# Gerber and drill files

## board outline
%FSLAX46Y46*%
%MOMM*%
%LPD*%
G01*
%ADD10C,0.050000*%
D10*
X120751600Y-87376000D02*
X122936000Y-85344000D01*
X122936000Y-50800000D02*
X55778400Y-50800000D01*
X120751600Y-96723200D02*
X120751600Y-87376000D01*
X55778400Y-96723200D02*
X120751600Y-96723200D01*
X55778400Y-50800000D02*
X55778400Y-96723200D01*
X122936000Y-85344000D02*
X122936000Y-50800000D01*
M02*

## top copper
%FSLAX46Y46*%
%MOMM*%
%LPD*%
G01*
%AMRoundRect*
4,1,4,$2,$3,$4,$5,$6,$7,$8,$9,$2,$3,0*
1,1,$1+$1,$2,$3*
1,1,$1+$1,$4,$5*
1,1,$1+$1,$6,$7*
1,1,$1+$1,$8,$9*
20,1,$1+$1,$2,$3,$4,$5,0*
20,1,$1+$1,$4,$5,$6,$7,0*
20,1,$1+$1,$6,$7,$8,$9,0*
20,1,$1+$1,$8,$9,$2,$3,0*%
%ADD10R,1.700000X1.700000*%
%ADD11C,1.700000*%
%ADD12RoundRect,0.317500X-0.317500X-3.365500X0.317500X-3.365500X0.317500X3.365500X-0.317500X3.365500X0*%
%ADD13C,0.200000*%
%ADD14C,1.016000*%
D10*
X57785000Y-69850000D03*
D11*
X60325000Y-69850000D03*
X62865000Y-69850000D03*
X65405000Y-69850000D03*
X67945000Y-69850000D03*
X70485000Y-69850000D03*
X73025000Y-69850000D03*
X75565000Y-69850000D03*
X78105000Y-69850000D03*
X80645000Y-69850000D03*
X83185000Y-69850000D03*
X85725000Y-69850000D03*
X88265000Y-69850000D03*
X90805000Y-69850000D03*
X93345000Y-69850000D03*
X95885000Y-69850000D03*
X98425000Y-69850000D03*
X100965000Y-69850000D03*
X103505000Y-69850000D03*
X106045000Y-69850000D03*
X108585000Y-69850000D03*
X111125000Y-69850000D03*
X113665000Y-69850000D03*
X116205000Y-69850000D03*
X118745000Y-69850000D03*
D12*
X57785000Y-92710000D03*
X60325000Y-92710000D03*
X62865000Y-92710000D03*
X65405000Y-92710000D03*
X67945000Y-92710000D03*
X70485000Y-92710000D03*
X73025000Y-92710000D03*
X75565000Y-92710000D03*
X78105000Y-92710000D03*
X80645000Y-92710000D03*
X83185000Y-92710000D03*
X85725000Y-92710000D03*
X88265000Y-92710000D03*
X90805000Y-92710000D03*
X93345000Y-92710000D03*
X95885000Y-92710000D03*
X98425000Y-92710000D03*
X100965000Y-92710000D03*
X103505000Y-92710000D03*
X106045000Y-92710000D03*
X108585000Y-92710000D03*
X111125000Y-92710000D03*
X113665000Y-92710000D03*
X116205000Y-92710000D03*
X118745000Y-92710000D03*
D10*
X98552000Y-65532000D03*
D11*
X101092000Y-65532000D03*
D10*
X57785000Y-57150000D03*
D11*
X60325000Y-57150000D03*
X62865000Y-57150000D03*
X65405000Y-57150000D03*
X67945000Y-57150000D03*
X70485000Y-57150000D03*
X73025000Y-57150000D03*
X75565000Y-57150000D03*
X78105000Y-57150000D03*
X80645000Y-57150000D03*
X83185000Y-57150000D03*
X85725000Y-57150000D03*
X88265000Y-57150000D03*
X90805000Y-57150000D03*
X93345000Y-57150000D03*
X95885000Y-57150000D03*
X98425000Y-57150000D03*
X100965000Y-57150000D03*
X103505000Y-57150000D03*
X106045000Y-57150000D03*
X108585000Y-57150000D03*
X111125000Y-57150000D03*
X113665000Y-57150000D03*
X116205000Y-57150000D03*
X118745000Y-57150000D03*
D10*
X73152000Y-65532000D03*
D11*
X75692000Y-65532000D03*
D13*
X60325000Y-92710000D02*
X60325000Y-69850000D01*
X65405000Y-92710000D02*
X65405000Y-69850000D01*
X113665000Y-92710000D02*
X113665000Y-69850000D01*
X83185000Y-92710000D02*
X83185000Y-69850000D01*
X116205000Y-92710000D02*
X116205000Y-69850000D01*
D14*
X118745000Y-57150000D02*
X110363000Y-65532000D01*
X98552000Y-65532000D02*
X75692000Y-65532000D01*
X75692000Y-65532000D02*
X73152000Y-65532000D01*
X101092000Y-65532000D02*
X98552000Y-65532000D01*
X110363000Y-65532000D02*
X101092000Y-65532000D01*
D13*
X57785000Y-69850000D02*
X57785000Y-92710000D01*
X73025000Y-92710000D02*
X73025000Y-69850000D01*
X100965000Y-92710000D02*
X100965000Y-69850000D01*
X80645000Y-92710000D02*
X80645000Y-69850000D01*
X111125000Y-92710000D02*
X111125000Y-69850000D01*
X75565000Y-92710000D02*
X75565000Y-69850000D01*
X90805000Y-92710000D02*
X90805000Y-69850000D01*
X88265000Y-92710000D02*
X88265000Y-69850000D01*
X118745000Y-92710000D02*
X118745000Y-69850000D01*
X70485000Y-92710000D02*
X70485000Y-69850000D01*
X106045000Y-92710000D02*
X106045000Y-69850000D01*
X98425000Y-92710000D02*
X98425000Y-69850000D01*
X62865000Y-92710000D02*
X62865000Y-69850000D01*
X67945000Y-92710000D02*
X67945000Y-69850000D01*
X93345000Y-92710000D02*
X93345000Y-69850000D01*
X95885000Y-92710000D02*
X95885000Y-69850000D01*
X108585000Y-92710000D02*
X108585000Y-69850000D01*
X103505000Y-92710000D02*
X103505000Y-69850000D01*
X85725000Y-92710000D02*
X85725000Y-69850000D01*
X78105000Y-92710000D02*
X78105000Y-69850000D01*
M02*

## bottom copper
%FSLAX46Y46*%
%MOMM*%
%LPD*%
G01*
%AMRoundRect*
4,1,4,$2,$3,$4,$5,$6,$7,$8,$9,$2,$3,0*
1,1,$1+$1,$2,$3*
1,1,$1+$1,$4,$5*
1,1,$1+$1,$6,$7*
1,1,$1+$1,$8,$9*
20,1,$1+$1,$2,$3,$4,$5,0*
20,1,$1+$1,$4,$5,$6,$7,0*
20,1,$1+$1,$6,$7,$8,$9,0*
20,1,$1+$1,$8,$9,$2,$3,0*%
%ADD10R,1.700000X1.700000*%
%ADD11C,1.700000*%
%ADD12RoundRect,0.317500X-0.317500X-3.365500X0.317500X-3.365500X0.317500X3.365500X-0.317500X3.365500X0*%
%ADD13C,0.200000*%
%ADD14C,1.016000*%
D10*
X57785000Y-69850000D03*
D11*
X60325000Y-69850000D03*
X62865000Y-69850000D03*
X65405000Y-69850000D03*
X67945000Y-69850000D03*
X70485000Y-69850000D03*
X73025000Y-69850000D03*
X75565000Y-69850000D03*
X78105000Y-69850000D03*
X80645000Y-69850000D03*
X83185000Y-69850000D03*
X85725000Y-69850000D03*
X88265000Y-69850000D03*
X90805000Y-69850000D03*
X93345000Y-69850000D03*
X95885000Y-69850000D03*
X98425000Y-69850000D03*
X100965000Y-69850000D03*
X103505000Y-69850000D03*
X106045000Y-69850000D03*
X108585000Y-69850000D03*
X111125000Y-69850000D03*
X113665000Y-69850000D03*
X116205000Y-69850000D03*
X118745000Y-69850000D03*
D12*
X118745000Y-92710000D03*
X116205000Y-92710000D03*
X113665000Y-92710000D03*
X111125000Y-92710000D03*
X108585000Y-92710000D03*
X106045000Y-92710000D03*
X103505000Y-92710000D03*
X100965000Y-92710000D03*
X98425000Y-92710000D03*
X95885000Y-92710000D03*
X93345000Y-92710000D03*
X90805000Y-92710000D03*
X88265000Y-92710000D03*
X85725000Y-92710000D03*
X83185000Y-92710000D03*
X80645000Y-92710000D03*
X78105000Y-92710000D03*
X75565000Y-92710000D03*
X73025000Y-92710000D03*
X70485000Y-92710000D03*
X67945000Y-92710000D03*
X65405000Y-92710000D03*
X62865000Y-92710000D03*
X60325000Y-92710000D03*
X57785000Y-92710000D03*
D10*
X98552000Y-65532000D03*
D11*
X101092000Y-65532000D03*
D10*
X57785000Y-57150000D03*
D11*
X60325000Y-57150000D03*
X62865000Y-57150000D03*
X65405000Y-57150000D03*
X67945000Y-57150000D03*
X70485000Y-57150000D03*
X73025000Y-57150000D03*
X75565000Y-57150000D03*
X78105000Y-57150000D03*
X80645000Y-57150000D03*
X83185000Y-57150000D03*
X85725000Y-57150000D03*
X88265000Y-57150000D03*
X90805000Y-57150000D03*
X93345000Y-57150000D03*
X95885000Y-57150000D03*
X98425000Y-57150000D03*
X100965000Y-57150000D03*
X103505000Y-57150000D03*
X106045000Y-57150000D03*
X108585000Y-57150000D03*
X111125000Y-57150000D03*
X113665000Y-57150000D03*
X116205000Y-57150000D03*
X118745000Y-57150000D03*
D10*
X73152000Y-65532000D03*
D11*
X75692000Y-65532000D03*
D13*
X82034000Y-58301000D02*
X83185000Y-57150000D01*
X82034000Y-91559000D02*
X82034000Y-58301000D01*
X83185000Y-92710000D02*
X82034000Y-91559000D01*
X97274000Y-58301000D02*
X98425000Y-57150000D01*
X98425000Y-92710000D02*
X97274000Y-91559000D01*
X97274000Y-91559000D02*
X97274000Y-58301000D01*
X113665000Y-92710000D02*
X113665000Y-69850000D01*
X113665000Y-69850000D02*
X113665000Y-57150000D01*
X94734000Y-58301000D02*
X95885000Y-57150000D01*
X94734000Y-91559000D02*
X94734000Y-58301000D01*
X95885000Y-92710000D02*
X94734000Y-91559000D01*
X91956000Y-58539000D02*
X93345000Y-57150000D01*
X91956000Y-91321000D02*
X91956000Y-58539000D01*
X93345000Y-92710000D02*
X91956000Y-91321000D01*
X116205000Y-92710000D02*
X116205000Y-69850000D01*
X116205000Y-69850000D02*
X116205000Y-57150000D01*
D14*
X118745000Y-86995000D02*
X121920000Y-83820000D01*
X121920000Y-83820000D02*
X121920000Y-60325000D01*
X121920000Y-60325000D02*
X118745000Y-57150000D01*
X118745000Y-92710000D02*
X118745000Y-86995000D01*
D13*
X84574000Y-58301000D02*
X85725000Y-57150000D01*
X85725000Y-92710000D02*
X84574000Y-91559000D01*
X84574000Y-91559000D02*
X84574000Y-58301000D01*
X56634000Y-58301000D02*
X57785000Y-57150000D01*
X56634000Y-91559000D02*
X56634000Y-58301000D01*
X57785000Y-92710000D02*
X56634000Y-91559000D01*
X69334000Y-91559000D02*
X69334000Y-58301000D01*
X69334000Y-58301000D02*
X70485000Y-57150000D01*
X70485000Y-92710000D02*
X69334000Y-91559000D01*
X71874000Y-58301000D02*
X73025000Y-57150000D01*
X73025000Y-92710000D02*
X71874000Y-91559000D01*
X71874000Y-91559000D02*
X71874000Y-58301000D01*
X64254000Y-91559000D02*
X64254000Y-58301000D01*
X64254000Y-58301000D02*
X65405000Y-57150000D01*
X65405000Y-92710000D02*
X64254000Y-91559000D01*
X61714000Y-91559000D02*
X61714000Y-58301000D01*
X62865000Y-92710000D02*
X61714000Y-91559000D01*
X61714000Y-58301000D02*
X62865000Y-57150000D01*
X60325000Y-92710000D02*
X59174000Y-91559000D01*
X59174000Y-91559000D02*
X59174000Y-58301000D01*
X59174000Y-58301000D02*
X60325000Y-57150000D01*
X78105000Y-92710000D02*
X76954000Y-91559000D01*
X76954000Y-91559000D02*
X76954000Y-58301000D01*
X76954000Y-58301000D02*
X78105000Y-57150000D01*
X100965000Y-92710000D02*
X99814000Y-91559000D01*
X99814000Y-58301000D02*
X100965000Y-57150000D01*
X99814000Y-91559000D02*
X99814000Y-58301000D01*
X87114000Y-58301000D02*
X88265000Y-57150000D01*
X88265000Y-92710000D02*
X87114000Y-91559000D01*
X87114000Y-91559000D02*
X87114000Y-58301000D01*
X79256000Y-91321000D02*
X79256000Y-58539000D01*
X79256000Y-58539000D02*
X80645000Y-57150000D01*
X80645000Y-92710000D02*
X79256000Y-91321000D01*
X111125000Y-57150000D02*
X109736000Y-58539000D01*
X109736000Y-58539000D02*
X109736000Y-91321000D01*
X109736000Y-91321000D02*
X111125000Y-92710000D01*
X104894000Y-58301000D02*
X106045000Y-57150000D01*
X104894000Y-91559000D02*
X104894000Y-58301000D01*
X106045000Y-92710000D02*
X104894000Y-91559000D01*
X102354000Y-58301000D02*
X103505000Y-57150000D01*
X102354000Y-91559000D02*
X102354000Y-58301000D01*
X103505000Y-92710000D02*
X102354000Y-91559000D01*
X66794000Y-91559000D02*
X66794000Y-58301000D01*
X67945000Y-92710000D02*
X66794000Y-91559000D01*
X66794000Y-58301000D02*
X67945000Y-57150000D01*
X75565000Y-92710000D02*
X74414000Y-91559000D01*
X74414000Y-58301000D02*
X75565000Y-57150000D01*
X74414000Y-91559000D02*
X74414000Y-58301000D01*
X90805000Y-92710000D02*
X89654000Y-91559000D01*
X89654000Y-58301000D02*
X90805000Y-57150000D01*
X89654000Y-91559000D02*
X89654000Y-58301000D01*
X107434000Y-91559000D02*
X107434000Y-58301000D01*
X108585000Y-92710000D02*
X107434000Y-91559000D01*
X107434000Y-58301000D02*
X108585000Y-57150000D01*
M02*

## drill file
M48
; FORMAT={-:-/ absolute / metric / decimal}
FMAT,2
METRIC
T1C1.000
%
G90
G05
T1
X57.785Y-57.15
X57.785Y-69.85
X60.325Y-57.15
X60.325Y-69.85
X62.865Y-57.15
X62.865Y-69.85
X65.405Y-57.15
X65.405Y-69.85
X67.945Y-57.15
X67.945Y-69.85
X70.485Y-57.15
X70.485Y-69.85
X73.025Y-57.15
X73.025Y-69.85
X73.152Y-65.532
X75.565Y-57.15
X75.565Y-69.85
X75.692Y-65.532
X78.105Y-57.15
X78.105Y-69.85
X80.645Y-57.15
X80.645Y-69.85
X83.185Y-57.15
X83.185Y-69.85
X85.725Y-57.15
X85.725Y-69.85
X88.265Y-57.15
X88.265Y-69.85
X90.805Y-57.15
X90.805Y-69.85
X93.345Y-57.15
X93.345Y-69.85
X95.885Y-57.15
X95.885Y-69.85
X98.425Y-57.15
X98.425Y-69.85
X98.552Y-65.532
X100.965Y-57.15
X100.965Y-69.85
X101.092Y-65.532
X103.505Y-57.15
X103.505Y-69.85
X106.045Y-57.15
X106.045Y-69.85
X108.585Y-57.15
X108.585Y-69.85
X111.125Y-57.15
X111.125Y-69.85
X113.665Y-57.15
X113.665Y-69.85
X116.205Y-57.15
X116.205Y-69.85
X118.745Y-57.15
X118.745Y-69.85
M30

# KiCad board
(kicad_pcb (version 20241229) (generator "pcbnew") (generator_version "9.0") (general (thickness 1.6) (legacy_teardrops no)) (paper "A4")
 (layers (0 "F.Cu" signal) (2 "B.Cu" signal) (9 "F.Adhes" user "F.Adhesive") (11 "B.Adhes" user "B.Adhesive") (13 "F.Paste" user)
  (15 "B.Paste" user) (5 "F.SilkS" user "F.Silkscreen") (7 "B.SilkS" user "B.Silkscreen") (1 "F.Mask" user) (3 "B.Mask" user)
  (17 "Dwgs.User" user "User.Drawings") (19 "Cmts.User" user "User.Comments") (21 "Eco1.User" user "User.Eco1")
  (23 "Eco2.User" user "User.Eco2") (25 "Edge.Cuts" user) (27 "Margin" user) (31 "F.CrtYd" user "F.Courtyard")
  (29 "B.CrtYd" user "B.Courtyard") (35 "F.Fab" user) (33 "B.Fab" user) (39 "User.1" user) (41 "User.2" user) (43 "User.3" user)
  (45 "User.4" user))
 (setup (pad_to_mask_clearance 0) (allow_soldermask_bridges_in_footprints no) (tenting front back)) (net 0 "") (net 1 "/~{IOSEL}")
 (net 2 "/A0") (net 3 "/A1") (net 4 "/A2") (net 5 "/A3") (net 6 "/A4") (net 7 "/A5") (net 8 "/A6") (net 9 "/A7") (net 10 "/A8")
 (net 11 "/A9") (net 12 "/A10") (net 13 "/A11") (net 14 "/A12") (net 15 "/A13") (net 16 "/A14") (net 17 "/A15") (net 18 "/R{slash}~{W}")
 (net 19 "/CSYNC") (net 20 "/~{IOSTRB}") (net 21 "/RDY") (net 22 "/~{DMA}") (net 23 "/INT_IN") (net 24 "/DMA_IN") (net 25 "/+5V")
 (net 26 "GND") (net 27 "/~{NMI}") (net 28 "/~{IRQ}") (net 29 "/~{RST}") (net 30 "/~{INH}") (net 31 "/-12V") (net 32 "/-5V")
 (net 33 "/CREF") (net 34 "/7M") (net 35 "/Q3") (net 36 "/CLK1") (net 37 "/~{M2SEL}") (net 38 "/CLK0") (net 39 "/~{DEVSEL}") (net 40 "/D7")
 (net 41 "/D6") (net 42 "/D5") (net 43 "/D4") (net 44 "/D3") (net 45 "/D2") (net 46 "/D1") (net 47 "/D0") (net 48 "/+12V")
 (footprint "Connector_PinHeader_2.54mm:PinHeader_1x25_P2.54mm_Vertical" (layer "F.Cu") (at 57.785 69.85 90)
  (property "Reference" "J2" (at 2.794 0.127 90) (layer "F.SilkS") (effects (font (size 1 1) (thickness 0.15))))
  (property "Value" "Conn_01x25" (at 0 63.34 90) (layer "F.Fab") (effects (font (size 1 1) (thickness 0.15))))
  (pad "1" thru_hole rect (at 0 0 90) (size 1.7 1.7) (drill 1) (layers "*.Cu" "*.Mask") (remove_unused_layers no) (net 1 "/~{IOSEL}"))
  (pad "2" thru_hole circle (at 0 2.54 90) (size 1.7 1.7) (drill 1) (layers "*.Cu" "*.Mask") (remove_unused_layers no) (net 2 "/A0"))
  (pad "3" thru_hole circle (at 0 5.08 90) (size 1.7 1.7) (drill 1) (layers "*.Cu" "*.Mask") (remove_unused_layers no) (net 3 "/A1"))
  (pad "4" thru_hole circle (at 0 7.62 90) (size 1.7 1.7) (drill 1) (layers "*.Cu" "*.Mask") (remove_unused_layers no) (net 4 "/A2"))
  (pad "5" thru_hole circle (at 0 10.16 90) (size 1.7 1.7) (drill 1) (layers "*.Cu" "*.Mask") (remove_unused_layers no) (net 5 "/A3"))
  (pad "6" thru_hole circle (at 0 12.7 90) (size 1.7 1.7) (drill 1) (layers "*.Cu" "*.Mask") (remove_unused_layers no) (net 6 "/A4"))
  (pad "7" thru_hole circle (at 0 15.24 90) (size 1.7 1.7) (drill 1) (layers "*.Cu" "*.Mask") (remove_unused_layers no) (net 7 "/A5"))
  (pad "8" thru_hole circle (at 0 17.78 90) (size 1.7 1.7) (drill 1) (layers "*.Cu" "*.Mask") (remove_unused_layers no) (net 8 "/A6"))
  (pad "9" thru_hole circle (at 0 20.32 90) (size 1.7 1.7) (drill 1) (layers "*.Cu" "*.Mask") (remove_unused_layers no) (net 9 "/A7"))
  (pad "10" thru_hole circle (at 0 22.86 90) (size 1.7 1.7) (drill 1) (layers "*.Cu" "*.Mask") (remove_unused_layers no) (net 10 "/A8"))
  (pad "11" thru_hole circle (at 0 25.4 90) (size 1.7 1.7) (drill 1) (layers "*.Cu" "*.Mask") (remove_unused_layers no) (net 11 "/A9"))
  (pad "12" thru_hole circle (at 0 27.94 90) (size 1.7 1.7) (drill 1) (layers "*.Cu" "*.Mask") (remove_unused_layers no) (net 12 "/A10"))
  (pad "13" thru_hole circle (at 0 30.48 90) (size 1.7 1.7) (drill 1) (layers "*.Cu" "*.Mask") (remove_unused_layers no) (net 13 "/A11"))
  (pad "14" thru_hole circle (at 0 33.02 90) (size 1.7 1.7) (drill 1) (layers "*.Cu" "*.Mask") (remove_unused_layers no) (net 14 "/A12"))
  (pad "15" thru_hole circle (at 0 35.56 90) (size 1.7 1.7) (drill 1) (layers "*.Cu" "*.Mask") (remove_unused_layers no) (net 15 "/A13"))
  (pad "16" thru_hole circle (at 0 38.1 90) (size 1.7 1.7) (drill 1) (layers "*.Cu" "*.Mask") (remove_unused_layers no) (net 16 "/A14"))
  (pad "17" thru_hole circle (at 0 40.64 90) (size 1.7 1.7) (drill 1) (layers "*.Cu" "*.Mask") (remove_unused_layers no) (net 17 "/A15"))
  (pad "18" thru_hole circle (at 0 43.18 90) (size 1.7 1.7) (drill 1) (layers "*.Cu" "*.Mask") (remove_unused_layers no)
   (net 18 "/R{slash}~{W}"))
  (pad "19" thru_hole circle (at 0 45.72 90) (size 1.7 1.7) (drill 1) (layers "*.Cu" "*.Mask") (remove_unused_layers no) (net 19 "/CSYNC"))
  (pad "20" thru_hole circle (at 0 48.26 90) (size 1.7 1.7) (drill 1) (layers "*.Cu" "*.Mask") (remove_unused_layers no)
   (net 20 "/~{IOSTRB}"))
  (pad "21" thru_hole circle (at 0 50.8 90) (size 1.7 1.7) (drill 1) (layers "*.Cu" "*.Mask") (remove_unused_layers no) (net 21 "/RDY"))
  (pad "22" thru_hole circle (at 0 53.34 90) (size 1.7 1.7) (drill 1) (layers "*.Cu" "*.Mask") (remove_unused_layers no) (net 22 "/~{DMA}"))
  (pad "23" thru_hole circle (at 0 55.88 90) (size 1.7 1.7) (drill 1) (layers "*.Cu" "*.Mask") (remove_unused_layers no) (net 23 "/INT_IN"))
  (pad "24" thru_hole circle (at 0 58.42 90) (size 1.7 1.7) (drill 1) (layers "*.Cu" "*.Mask") (remove_unused_layers no) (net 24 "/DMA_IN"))
  (pad "25" thru_hole circle (at 0 60.96 90) (size 1.7 1.7) (drill 1) (layers "*.Cu" "*.Mask") (remove_unused_layers no) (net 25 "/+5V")))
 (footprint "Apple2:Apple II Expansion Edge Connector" (layer "F.Cu") (at 71.755 87.757)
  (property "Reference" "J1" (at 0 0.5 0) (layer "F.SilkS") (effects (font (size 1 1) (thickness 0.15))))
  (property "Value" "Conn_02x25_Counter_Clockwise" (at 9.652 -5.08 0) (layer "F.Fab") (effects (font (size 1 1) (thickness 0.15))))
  (pad "1" connect roundrect (at -13.97 4.953) (size 1.27 7.366) (layers "F.Cu" "F.Mask") (roundrect_rratio 0.25) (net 1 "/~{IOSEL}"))
  (pad "2" connect roundrect (at -11.43 4.953) (size 1.27 7.366) (layers "F.Cu" "F.Mask") (roundrect_rratio 0.25) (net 2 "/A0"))
  (pad "3" connect roundrect (at -8.89 4.953) (size 1.27 7.366) (layers "F.Cu" "F.Mask") (roundrect_rratio 0.25) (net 3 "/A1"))
  (pad "4" connect roundrect (at -6.35 4.953) (size 1.27 7.366) (layers "F.Cu" "F.Mask") (roundrect_rratio 0.25) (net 4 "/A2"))
  (pad "5" connect roundrect (at -3.81 4.953) (size 1.27 7.366) (layers "F.Cu" "F.Mask") (roundrect_rratio 0.25) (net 5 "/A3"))
  (pad "6" connect roundrect (at -1.27 4.953) (size 1.27 7.366) (layers "F.Cu" "F.Mask") (roundrect_rratio 0.25) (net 6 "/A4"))
  (pad "7" connect roundrect (at 1.27 4.953) (size 1.27 7.366) (layers "F.Cu" "F.Mask") (roundrect_rratio 0.25) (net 7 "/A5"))
  (pad "8" connect roundrect (at 3.81 4.953) (size 1.27 7.366) (layers "F.Cu" "F.Mask") (roundrect_rratio 0.25) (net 8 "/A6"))
  (pad "9" connect roundrect (at 6.35 4.953) (size 1.27 7.366) (layers "F.Cu" "F.Mask") (roundrect_rratio 0.25) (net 9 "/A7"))
  (pad "10" connect roundrect (at 8.89 4.953) (size 1.27 7.366) (layers "F.Cu" "F.Mask") (roundrect_rratio 0.25) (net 10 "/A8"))
  (pad "11" connect roundrect (at 11.43 4.953) (size 1.27 7.366) (layers "F.Cu" "F.Mask") (roundrect_rratio 0.25) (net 11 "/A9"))
  (pad "12" connect roundrect (at 13.97 4.953) (size 1.27 7.366) (layers "F.Cu" "F.Mask") (roundrect_rratio 0.25) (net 12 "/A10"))
  (pad "13" connect roundrect (at 16.51 4.953) (size 1.27 7.366) (layers "F.Cu" "F.Mask") (roundrect_rratio 0.25) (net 13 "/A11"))
  (pad "14" connect roundrect (at 19.05 4.953) (size 1.27 7.366) (layers "F.Cu" "F.Mask") (roundrect_rratio 0.25) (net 14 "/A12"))
  (pad "15" connect roundrect (at 21.59 4.953) (size 1.27 7.366) (layers "F.Cu" "F.Mask") (roundrect_rratio 0.25) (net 15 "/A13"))
  (pad "16" connect roundrect (at 24.13 4.953) (size 1.27 7.366) (layers "F.Cu" "F.Mask") (roundrect_rratio 0.25) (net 16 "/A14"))
  (pad "17" connect roundrect (at 26.67 4.953) (size 1.27 7.366) (layers "F.Cu" "F.Mask") (roundrect_rratio 0.25) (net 17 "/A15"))
  (pad "18" connect roundrect (at 29.21 4.953) (size 1.27 7.366) (layers "F.Cu" "F.Mask") (roundrect_rratio 0.25) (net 18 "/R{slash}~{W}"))
  (pad "19" connect roundrect (at 31.75 4.953) (size 1.27 7.366) (layers "F.Cu" "F.Mask") (roundrect_rratio 0.25) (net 19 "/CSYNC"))
  (pad "20" connect roundrect (at 34.29 4.953) (size 1.27 7.366) (layers "F.Cu" "F.Mask") (roundrect_rratio 0.25) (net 20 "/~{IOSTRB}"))
  (pad "21" connect roundrect (at 36.83 4.953) (size 1.27 7.366) (layers "F.Cu" "F.Mask") (roundrect_rratio 0.25) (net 21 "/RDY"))
  (pad "22" connect roundrect (at 39.37 4.953) (size 1.27 7.366) (layers "F.Cu" "F.Mask") (roundrect_rratio 0.25) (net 22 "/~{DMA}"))
  (pad "23" connect roundrect (at 41.91 4.953) (size 1.27 7.366) (layers "F.Cu" "F.Mask") (roundrect_rratio 0.25) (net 23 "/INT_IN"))
  (pad "24" connect roundrect (at 44.45 4.953) (size 1.27 7.366) (layers "F.Cu" "F.Mask") (roundrect_rratio 0.25) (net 24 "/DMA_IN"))
  (pad "25" connect roundrect (at 46.99 4.953) (size 1.27 7.366) (layers "F.Cu" "F.Mask") (roundrect_rratio 0.25) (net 25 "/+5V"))
  (pad "26" connect roundrect (at 46.99 4.953) (size 1.27 7.366) (layers "B.Cu" "B.Mask") (roundrect_rratio 0.25) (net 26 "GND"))
  (pad "27" connect roundrect (at 44.45 4.953) (size 1.27 7.366) (layers "B.Cu" "B.Mask") (roundrect_rratio 0.25) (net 24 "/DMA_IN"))
  (pad "28" connect roundrect (at 41.91 4.953) (size 1.27 7.366) (layers "B.Cu" "B.Mask") (roundrect_rratio 0.25) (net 23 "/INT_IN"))
  (pad "29" connect roundrect (at 39.37 4.953) (size 1.27 7.366) (layers "B.Cu" "B.Mask") (roundrect_rratio 0.25) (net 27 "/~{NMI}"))
  (pad "30" connect roundrect (at 36.83 4.953) (size 1.27 7.366) (layers "B.Cu" "B.Mask") (roundrect_rratio 0.25) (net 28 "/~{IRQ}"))
  (pad "31" connect roundrect (at 34.29 4.953) (size 1.27 7.366) (layers "B.Cu" "B.Mask") (roundrect_rratio 0.25) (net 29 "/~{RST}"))
  (pad "32" connect roundrect (at 31.75 4.953) (size 1.27 7.366) (layers "B.Cu" "B.Mask") (roundrect_rratio 0.25) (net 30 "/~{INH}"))
  (pad "33" connect roundrect (at 29.21 4.953) (size 1.27 7.366) (layers "B.Cu" "B.Mask") (roundrect_rratio 0.25) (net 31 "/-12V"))
  (pad "34" connect roundrect (at 26.67 4.953) (size 1.27 7.366) (layers "B.Cu" "B.Mask") (roundrect_rratio 0.25) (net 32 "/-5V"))
  (pad "35" connect roundrect (at 24.13 4.953) (size 1.27 7.366) (layers "B.Cu" "B.Mask") (roundrect_rratio 0.25) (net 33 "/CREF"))
  (pad "36" connect roundrect (at 21.59 4.953) (size 1.27 7.366) (layers "B.Cu" "B.Mask") (roundrect_rratio 0.25) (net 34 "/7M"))
  (pad "37" connect roundrect (at 19.05 4.953) (size 1.27 7.366) (layers "B.Cu" "B.Mask") (roundrect_rratio 0.25) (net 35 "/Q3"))
  (pad "38" connect roundrect (at 16.51 4.953) (size 1.27 7.366) (layers "B.Cu" "B.Mask") (roundrect_rratio 0.25) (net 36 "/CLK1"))
  (pad "39" connect roundrect (at 13.97 4.953) (size 1.27 7.366) (layers "B.Cu" "B.Mask") (roundrect_rratio 0.25) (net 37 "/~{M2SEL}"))
  (pad "40" connect roundrect (at 11.43 4.953) (size 1.27 7.366) (layers "B.Cu" "B.Mask") (roundrect_rratio 0.25) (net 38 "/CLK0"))
  (pad "41" connect roundrect (at 8.89 4.953) (size 1.27 7.366) (layers "B.Cu" "B.Mask") (roundrect_rratio 0.25) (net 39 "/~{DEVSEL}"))
  (pad "42" connect roundrect (at 6.35 4.953) (size 1.27 7.366) (layers "B.Cu" "B.Mask") (roundrect_rratio 0.25) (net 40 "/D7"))
  (pad "43" connect roundrect (at 3.81 4.953) (size 1.27 7.366) (layers "B.Cu" "B.Mask") (roundrect_rratio 0.25) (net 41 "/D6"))
  (pad "44" connect roundrect (at 1.27 4.953) (size 1.27 7.366) (layers "B.Cu" "B.Mask") (roundrect_rratio 0.25) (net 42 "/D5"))
  (pad "45" connect roundrect (at -1.27 4.953) (size 1.27 7.366) (layers "B.Cu" "B.Mask") (roundrect_rratio 0.25) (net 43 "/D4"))
  (pad "46" connect roundrect (at -3.81 4.953) (size 1.27 7.366) (layers "B.Cu" "B.Mask") (roundrect_rratio 0.25) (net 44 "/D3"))
  (pad "47" connect roundrect (at -6.35 4.953) (size 1.27 7.366) (layers "B.Cu" "B.Mask") (roundrect_rratio 0.25) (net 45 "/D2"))
  (pad "48" connect roundrect (at -8.89 4.953) (size 1.27 7.366) (layers "B.Cu" "B.Mask") (roundrect_rratio 0.25) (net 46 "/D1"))
  (pad "49" connect roundrect (at -11.43 4.953) (size 1.27 7.366) (layers "B.Cu" "B.Mask") (roundrect_rratio 0.25) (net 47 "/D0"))
  (pad "50" connect roundrect (at -13.97 4.953) (size 1.27 7.366) (layers "B.Cu" "B.Mask") (roundrect_rratio 0.25) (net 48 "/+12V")))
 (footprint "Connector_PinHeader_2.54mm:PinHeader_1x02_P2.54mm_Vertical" (layer "F.Cu") (at 98.552 65.532 90)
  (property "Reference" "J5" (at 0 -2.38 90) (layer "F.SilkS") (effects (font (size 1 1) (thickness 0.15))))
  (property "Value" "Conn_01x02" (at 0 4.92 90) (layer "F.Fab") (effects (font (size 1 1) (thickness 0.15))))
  (pad "1" thru_hole rect (at 0 0 90) (size 1.7 1.7) (drill 1) (layers "*.Cu" "*.Mask") (remove_unused_layers no) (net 26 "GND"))
  (pad "2" thru_hole circle (at 0 2.54 90) (size 1.7 1.7) (drill 1) (layers "*.Cu" "*.Mask") (remove_unused_layers no) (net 26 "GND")))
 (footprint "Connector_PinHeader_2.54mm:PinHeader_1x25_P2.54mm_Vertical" (layer "F.Cu") (at 57.785 57.15 90)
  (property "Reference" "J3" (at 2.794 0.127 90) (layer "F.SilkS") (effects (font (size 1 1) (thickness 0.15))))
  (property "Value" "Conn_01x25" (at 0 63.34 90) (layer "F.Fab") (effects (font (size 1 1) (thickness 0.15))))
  (pad "1" thru_hole rect (at 0 0 90) (size 1.7 1.7) (drill 1) (layers "*.Cu" "*.Mask") (remove_unused_layers no) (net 48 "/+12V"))
  (pad "2" thru_hole circle (at 0 2.54 90) (size 1.7 1.7) (drill 1) (layers "*.Cu" "*.Mask") (remove_unused_layers no) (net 47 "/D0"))
  (pad "3" thru_hole circle (at 0 5.08 90) (size 1.7 1.7) (drill 1) (layers "*.Cu" "*.Mask") (remove_unused_layers no) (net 46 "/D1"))
  (pad "4" thru_hole circle (at 0 7.62 90) (size 1.7 1.7) (drill 1) (layers "*.Cu" "*.Mask") (remove_unused_layers no) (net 45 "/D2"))
  (pad "5" thru_hole circle (at 0 10.16 90) (size 1.7 1.7) (drill 1) (layers "*.Cu" "*.Mask") (remove_unused_layers no) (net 44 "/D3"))
  (pad "6" thru_hole circle (at 0 12.7 90) (size 1.7 1.7) (drill 1) (layers "*.Cu" "*.Mask") (remove_unused_layers no) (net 43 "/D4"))
  (pad "7" thru_hole circle (at 0 15.24 90) (size 1.7 1.7) (drill 1) (layers "*.Cu" "*.Mask") (remove_unused_layers no) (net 42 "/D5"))
  (pad "8" thru_hole circle (at 0 17.78 90) (size 1.7 1.7) (drill 1) (layers "*.Cu" "*.Mask") (remove_unused_layers no) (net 41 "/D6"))
  (pad "9" thru_hole circle (at 0 20.32 90) (size 1.7 1.7) (drill 1) (layers "*.Cu" "*.Mask") (remove_unused_layers no) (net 40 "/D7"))
  (pad "10" thru_hole circle (at 0 22.86 90) (size 1.7 1.7) (drill 1) (layers "*.Cu" "*.Mask") (remove_unused_layers no)
   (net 39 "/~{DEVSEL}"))
  (pad "11" thru_hole circle (at 0 25.4 90) (size 1.7 1.7) (drill 1) (layers "*.Cu" "*.Mask") (remove_unused_layers no) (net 38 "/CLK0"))
  (pad "12" thru_hole circle (at 0 27.94 90) (size 1.7 1.7) (drill 1) (layers "*.Cu" "*.Mask") (remove_unused_layers no)
   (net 37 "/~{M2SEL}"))
  (pad "13" thru_hole circle (at 0 30.48 90) (size 1.7 1.7) (drill 1) (layers "*.Cu" "*.Mask") (remove_unused_layers no) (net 36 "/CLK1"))
  (pad "14" thru_hole circle (at 0 33.02 90) (size 1.7 1.7) (drill 1) (layers "*.Cu" "*.Mask") (remove_unused_layers no) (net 35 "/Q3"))
  (pad "15" thru_hole circle (at 0 35.56 90) (size 1.7 1.7) (drill 1) (layers "*.Cu" "*.Mask") (remove_unused_layers no) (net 34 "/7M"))
  (pad "16" thru_hole circle (at 0 38.1 90) (size 1.7 1.7) (drill 1) (layers "*.Cu" "*.Mask") (remove_unused_layers no) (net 33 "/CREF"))
  (pad "17" thru_hole circle (at 0 40.64 90) (size 1.7 1.7) (drill 1) (layers "*.Cu" "*.Mask") (remove_unused_layers no) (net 32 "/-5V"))
  (pad "18" thru_hole circle (at 0 43.18 90) (size 1.7 1.7) (drill 1) (layers "*.Cu" "*.Mask") (remove_unused_layers no) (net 31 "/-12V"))
  (pad "19" thru_hole circle (at 0 45.72 90) (size 1.7 1.7) (drill 1) (layers "*.Cu" "*.Mask") (remove_unused_layers no) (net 30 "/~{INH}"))
  (pad "20" thru_hole circle (at 0 48.26 90) (size 1.7 1.7) (drill 1) (layers "*.Cu" "*.Mask") (remove_unused_layers no) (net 29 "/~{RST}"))
  (pad "21" thru_hole circle (at 0 50.8 90) (size 1.7 1.7) (drill 1) (layers "*.Cu" "*.Mask") (remove_unused_layers no) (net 28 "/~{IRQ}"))
  (pad "22" thru_hole circle (at 0 53.34 90) (size 1.7 1.7) (drill 1) (layers "*.Cu" "*.Mask") (remove_unused_layers no) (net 27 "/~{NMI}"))
  (pad "23" thru_hole circle (at 0 55.88 90) (size 1.7 1.7) (drill 1) (layers "*.Cu" "*.Mask") (remove_unused_layers no) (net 23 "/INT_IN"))
  (pad "24" thru_hole circle (at 0 58.42 90) (size 1.7 1.7) (drill 1) (layers "*.Cu" "*.Mask") (remove_unused_layers no) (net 24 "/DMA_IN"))
  (pad "25" thru_hole circle (at 0 60.96 90) (size 1.7 1.7) (drill 1) (layers "*.Cu" "*.Mask") (remove_unused_layers no) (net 26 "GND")))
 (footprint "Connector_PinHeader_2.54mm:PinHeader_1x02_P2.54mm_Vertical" (layer "F.Cu") (at 73.152 65.532 90)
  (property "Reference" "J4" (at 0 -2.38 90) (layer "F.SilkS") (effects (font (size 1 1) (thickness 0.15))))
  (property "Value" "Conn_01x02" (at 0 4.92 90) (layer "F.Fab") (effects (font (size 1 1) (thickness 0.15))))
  (pad "1" thru_hole rect (at 0 0 90) (size 1.7 1.7) (drill 1) (layers "*.Cu" "*.Mask") (remove_unused_layers no) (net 26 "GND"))
  (pad "2" thru_hole circle (at 0 2.54 90) (size 1.7 1.7) (drill 1) (layers "*.Cu" "*.Mask") (remove_unused_layers no) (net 26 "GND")))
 (gr_line (start 120.7516 87.376) (end 122.936 85.344) (stroke (width 0.05) (type default)) (layer "Edge.Cuts"))
 (gr_line (start 122.936 50.8) (end 55.7784 50.8) (stroke (width 0.05) (type default)) (layer "Edge.Cuts"))
 (gr_line (start 120.7516 96.7232) (end 120.7516 87.376) (stroke (width 0.05) (type default)) (layer "Edge.Cuts"))
 (gr_line (start 55.7784 96.7232) (end 120.7516 96.7232) (stroke (width 0.05) (type default)) (layer "Edge.Cuts"))
 (gr_line (start 55.7784 50.8) (end 55.7784 96.7232) (stroke (width 0.05) (type default)) (layer "Edge.Cuts"))
 (gr_line (start 122.936 85.344) (end 122.936 50.8) (stroke (width 0.05) (type default)) (layer "Edge.Cuts"))
 (segment (start 60.325 92.71) (end 60.325 69.85) (width 0.2) (layer "F.Cu") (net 2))
 (segment (start 82.034 58.301) (end 83.185 57.15) (width 0.2) (layer "B.Cu") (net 38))
 (segment (start 82.034 91.559) (end 82.034 58.301) (width 0.2) (layer "B.Cu") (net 38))
 (segment (start 83.185 92.71) (end 82.034 91.559) (width 0.2) (layer "B.Cu") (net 38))
 (segment (start 97.274 58.301) (end 98.425 57.15) (width 0.2) (layer "B.Cu") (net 32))
 (segment (start 98.425 92.71) (end 97.274 91.559) (width 0.2) (layer "B.Cu") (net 32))
 (segment (start 97.274 91.559) (end 97.274 58.301) (width 0.2) (layer "B.Cu") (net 32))
 (segment (start 65.405 92.71) (end 65.405 69.85) (width 0.2) (layer "F.Cu") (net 4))
 (segment (start 113.665 92.71) (end 113.665 69.85) (width 0.2) (layer "F.Cu") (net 23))
 (segment (start 113.665 92.71) (end 113.665 69.85) (width 0.2) (layer "B.Cu") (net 23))
 (segment (start 113.665 69.85) (end 113.665 57.15) (width 0.2) (layer "B.Cu") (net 23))
 (segment (start 94.734 58.301) (end 95.885 57.15) (width 0.2) (layer "B.Cu") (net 33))
 (segment (start 94.734 91.559) (end 94.734 58.301) (width 0.2) (layer "B.Cu") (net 33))
 (segment (start 95.885 92.71) (end 94.734 91.559) (width 0.2) (layer "B.Cu") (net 33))
 (segment (start 83.185 92.71) (end 83.185 69.85) (width 0.2) (layer "F.Cu") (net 11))
 (segment (start 91.956 58.539) (end 93.345 57.15) (width 0.2) (layer "B.Cu") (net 34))
 (segment (start 91.956 91.321) (end 91.956 58.539) (width 0.2) (layer "B.Cu") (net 34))
 (segment (start 93.345 92.71) (end 91.956 91.321) (width 0.2) (layer "B.Cu") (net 34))
 (segment (start 116.205 92.71) (end 116.205 69.85) (width 0.2) (layer "F.Cu") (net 24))
 (segment (start 116.205 92.71) (end 116.205 69.85) (width 0.2) (layer "B.Cu") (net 24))
 (segment (start 116.205 69.85) (end 116.205 57.15) (width 0.2) (layer "B.Cu") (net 24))
 (segment (start 118.745 57.15) (end 110.363 65.532) (width 1.016) (layer "F.Cu") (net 26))
 (segment (start 98.552 65.532) (end 75.692 65.532) (width 1.016) (layer "F.Cu") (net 26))
 (segment (start 75.692 65.532) (end 73.152 65.532) (width 1.016) (layer "F.Cu") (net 26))
 (segment (start 101.092 65.532) (end 98.552 65.532) (width 1.016) (layer "F.Cu") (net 26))
 (segment (start 110.363 65.532) (end 101.092 65.532) (width 1.016) (layer "F.Cu") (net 26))
 (segment (start 118.745 86.995) (end 121.92 83.82) (width 1.016) (layer "B.Cu") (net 26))
 (segment (start 121.92 83.82) (end 121.92 60.325) (width 1.016) (layer "B.Cu") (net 26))
 (segment (start 121.92 60.325) (end 118.745 57.15) (width 1.016) (layer "B.Cu") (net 26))
 (segment (start 118.745 92.71) (end 118.745 86.995) (width 1.016) (layer "B.Cu") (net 26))
 (segment (start 84.574 58.301) (end 85.725 57.15) (width 0.2) (layer "B.Cu") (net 37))
 (segment (start 85.725 92.71) (end 84.574 91.559) (width 0.2) (layer "B.Cu") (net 37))
 (segment (start 84.574 91.559) (end 84.574 58.301) (width 0.2) (layer "B.Cu") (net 37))
 (segment (start 56.634 58.301) (end 57.785 57.15) (width 0.2) (layer "B.Cu") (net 48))
 (segment (start 56.634 91.559) (end 56.634 58.301) (width 0.2) (layer "B.Cu") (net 48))
 (segment (start 57.785 92.71) (end 56.634 91.559) (width 0.2) (layer "B.Cu") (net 48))
 (segment (start 57.785 69.85) (end 57.785 92.71) (width 0.2) (layer "F.Cu") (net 1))
 (segment (start 73.025 92.71) (end 73.025 69.85) (width 0.2) (layer "F.Cu") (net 7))
 (segment (start 100.965 92.71) (end 100.965 69.85) (width 0.2) (layer "F.Cu") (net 18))
 (segment (start 80.645 92.71) (end 80.645 69.85) (width 0.2) (layer "F.Cu") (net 10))
 (segment (start 111.125 92.71) (end 111.125 69.85) (width 0.2) (layer "F.Cu") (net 22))
 (segment (start 75.565 92.71) (end 75.565 69.85) (width 0.2) (layer "F.Cu") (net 8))
 (segment (start 90.805 92.71) (end 90.805 69.85) (width 0.2) (layer "F.Cu") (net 14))
 (segment (start 69.334 91.559) (end 69.334 58.301) (width 0.2) (layer "B.Cu") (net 43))
 (segment (start 69.334 58.301) (end 70.485 57.15) (width 0.2) (layer "B.Cu") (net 43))
 (segment (start 70.485 92.71) (end 69.334 91.559) (width 0.2) (layer "B.Cu") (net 43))
 (segment (start 71.874 58.301) (end 73.025 57.15) (width 0.2) (layer "B.Cu") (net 42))
 (segment (start 73.025 92.71) (end 71.874 91.559) (width 0.2) (layer "B.Cu") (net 42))
 (segment (start 71.874 91.559) (end 71.874 58.301) (width 0.2) (layer "B.Cu") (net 42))
 (segment (start 64.254 91.559) (end 64.254 58.301) (width 0.2) (layer "B.Cu") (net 45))
 (segment (start 64.254 58.301) (end 65.405 57.15) (width 0.2) (layer "B.Cu") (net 45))
 (segment (start 65.405 92.71) (end 64.254 91.559) (width 0.2) (layer "B.Cu") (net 45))
 (segment (start 61.714 91.559) (end 61.714 58.301) (width 0.2) (layer "B.Cu") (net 46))
 (segment (start 62.865 92.71) (end 61.714 91.559) (width 0.2) (layer "B.Cu") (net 46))
 (segment (start 61.714 58.301) (end 62.865 57.15) (width 0.2) (layer "B.Cu") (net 46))
 (segment (start 60.325 92.71) (end 59.174 91.559) (width 0.2) (layer "B.Cu") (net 47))
 (segment (start 59.174 91.559) (end 59.174 58.301) (width 0.2) (layer "B.Cu") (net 47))
 (segment (start 59.174 58.301) (end 60.325 57.15) (width 0.2) (layer "B.Cu") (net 47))
 (segment (start 88.265 92.71) (end 88.265 69.85) (width 0.2) (layer "F.Cu") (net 13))
 (segment (start 118.745 92.71) (end 118.745 69.85) (width 0.2) (layer "F.Cu") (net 25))
 (segment (start 70.485 92.71) (end 70.485 69.85) (width 0.2) (layer "F.Cu") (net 6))
 (segment (start 78.105 92.71) (end 76.954 91.559) (width 0.2) (layer "B.Cu") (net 40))
 (segment (start 76.954 91.559) (end 76.954 58.301) (width 0.2) (layer "B.Cu") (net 40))
 (segment (start 76.954 58.301) (end 78.105 57.15) (width 0.2) (layer "B.Cu") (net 40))
 (segment (start 100.965 92.71) (end 99.814 91.559) (width 0.2) (layer "B.Cu") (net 31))
 (segment (start 99.814 58.301) (end 100.965 57.15) (width 0.2) (layer "B.Cu") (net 31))
 (segment (start 99.814 91.559) (end 99.814 58.301) (width 0.2) (layer "B.Cu") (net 31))
 (segment (start 87.114 58.301) (end 88.265 57.15) (width 0.2) (layer "B.Cu") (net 36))
 (segment (start 88.265 92.71) (end 87.114 91.559) (width 0.2) (layer "B.Cu") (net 36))
 (segment (start 87.114 91.559) (end 87.114 58.301) (width 0.2) (layer "B.Cu") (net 36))
 (segment (start 106.045 92.71) (end 106.045 69.85) (width 0.2) (layer "F.Cu") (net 20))
 (segment (start 98.425 92.71) (end 98.425 69.85) (width 0.2) (layer "F.Cu") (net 17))
 (segment (start 62.865 92.71) (end 62.865 69.85) (width 0.2) (layer "F.Cu") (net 3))
 (segment (start 67.945 92.71) (end 67.945 69.85) (width 0.2) (layer "F.Cu") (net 5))
 (segment (start 93.345 92.71) (end 93.345 69.85) (width 0.2) (layer "F.Cu") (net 15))
 (segment (start 79.256 91.321) (end 79.256 58.539) (width 0.2) (layer "B.Cu") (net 39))
 (segment (start 79.256 58.539) (end 80.645 57.15) (width 0.2) (layer "B.Cu") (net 39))
 (segment (start 80.645 92.71) (end 79.256 91.321) (width 0.2) (layer "B.Cu") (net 39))
 (segment (start 111.125 57.15) (end 109.736 58.539) (width 0.2) (layer "B.Cu") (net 27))
 (segment (start 109.736 58.539) (end 109.736 91.321) (width 0.2) (layer "B.Cu") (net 27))
 (segment (start 109.736 91.321) (end 111.125 92.71) (width 0.2) (layer "B.Cu") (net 27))
 (segment (start 95.885 92.71) (end 95.885 69.85) (width 0.2) (layer "F.Cu") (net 16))
 (segment (start 108.585 92.71) (end 108.585 69.85) (width 0.2) (layer "F.Cu") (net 21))
 (segment (start 104.894 58.301) (end 106.045 57.15) (width 0.2) (layer "B.Cu") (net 29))
 (segment (start 104.894 91.559) (end 104.894 58.301) (width 0.2) (layer "B.Cu") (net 29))
 (segment (start 106.045 92.71) (end 104.894 91.559) (width 0.2) (layer "B.Cu") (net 29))
 (segment (start 102.354 58.301) (end 103.505 57.15) (width 0.2) (layer "B.Cu") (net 30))
 (segment (start 102.354 91.559) (end 102.354 58.301) (width 0.2) (layer "B.Cu") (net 30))
 (segment (start 103.505 92.71) (end 102.354 91.559) (width 0.2) (layer "B.Cu") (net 30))
 (segment (start 103.505 92.71) (end 103.505 69.85) (width 0.2) (layer "F.Cu") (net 19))
 (segment (start 66.794 91.559) (end 66.794 58.301) (width 0.2) (layer "B.Cu") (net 44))
 (segment (start 67.945 92.71) (end 66.794 91.559) (width 0.2) (layer "B.Cu") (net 44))
 (segment (start 66.794 58.301) (end 67.945 57.15) (width 0.2) (layer "B.Cu") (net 44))
 (segment (start 75.565 92.71) (end 74.414 91.559) (width 0.2) (layer "B.Cu") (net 41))
 (segment (start 74.414 58.301) (end 75.565 57.15) (width 0.2) (layer "B.Cu") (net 41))
 (segment (start 74.414 91.559) (end 74.414 58.301) (width 0.2) (layer "B.Cu") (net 41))
 (segment (start 90.805 92.71) (end 89.654 91.559) (width 0.2) (layer "B.Cu") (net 35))
 (segment (start 89.654 58.301) (end 90.805 57.15) (width 0.2) (layer "B.Cu") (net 35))
 (segment (start 89.654 91.559) (end 89.654 58.301) (width 0.2) (layer "B.Cu") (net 35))
 (segment (start 107.434 91.559) (end 107.434 58.301) (width 0.2) (layer "B.Cu") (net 28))
 (segment (start 108.585 92.71) (end 107.434 91.559) (width 0.2) (layer "B.Cu") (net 28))
 (segment (start 107.434 58.301) (end 108.585 57.15) (width 0.2) (layer "B.Cu") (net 28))
 (segment (start 85.725 92.71) (end 85.725 69.85) (width 0.2) (layer "F.Cu") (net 12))
 (segment (start 78.105 92.71) (end 78.105 69.85) (width 0.2) (layer "F.Cu") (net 9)))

